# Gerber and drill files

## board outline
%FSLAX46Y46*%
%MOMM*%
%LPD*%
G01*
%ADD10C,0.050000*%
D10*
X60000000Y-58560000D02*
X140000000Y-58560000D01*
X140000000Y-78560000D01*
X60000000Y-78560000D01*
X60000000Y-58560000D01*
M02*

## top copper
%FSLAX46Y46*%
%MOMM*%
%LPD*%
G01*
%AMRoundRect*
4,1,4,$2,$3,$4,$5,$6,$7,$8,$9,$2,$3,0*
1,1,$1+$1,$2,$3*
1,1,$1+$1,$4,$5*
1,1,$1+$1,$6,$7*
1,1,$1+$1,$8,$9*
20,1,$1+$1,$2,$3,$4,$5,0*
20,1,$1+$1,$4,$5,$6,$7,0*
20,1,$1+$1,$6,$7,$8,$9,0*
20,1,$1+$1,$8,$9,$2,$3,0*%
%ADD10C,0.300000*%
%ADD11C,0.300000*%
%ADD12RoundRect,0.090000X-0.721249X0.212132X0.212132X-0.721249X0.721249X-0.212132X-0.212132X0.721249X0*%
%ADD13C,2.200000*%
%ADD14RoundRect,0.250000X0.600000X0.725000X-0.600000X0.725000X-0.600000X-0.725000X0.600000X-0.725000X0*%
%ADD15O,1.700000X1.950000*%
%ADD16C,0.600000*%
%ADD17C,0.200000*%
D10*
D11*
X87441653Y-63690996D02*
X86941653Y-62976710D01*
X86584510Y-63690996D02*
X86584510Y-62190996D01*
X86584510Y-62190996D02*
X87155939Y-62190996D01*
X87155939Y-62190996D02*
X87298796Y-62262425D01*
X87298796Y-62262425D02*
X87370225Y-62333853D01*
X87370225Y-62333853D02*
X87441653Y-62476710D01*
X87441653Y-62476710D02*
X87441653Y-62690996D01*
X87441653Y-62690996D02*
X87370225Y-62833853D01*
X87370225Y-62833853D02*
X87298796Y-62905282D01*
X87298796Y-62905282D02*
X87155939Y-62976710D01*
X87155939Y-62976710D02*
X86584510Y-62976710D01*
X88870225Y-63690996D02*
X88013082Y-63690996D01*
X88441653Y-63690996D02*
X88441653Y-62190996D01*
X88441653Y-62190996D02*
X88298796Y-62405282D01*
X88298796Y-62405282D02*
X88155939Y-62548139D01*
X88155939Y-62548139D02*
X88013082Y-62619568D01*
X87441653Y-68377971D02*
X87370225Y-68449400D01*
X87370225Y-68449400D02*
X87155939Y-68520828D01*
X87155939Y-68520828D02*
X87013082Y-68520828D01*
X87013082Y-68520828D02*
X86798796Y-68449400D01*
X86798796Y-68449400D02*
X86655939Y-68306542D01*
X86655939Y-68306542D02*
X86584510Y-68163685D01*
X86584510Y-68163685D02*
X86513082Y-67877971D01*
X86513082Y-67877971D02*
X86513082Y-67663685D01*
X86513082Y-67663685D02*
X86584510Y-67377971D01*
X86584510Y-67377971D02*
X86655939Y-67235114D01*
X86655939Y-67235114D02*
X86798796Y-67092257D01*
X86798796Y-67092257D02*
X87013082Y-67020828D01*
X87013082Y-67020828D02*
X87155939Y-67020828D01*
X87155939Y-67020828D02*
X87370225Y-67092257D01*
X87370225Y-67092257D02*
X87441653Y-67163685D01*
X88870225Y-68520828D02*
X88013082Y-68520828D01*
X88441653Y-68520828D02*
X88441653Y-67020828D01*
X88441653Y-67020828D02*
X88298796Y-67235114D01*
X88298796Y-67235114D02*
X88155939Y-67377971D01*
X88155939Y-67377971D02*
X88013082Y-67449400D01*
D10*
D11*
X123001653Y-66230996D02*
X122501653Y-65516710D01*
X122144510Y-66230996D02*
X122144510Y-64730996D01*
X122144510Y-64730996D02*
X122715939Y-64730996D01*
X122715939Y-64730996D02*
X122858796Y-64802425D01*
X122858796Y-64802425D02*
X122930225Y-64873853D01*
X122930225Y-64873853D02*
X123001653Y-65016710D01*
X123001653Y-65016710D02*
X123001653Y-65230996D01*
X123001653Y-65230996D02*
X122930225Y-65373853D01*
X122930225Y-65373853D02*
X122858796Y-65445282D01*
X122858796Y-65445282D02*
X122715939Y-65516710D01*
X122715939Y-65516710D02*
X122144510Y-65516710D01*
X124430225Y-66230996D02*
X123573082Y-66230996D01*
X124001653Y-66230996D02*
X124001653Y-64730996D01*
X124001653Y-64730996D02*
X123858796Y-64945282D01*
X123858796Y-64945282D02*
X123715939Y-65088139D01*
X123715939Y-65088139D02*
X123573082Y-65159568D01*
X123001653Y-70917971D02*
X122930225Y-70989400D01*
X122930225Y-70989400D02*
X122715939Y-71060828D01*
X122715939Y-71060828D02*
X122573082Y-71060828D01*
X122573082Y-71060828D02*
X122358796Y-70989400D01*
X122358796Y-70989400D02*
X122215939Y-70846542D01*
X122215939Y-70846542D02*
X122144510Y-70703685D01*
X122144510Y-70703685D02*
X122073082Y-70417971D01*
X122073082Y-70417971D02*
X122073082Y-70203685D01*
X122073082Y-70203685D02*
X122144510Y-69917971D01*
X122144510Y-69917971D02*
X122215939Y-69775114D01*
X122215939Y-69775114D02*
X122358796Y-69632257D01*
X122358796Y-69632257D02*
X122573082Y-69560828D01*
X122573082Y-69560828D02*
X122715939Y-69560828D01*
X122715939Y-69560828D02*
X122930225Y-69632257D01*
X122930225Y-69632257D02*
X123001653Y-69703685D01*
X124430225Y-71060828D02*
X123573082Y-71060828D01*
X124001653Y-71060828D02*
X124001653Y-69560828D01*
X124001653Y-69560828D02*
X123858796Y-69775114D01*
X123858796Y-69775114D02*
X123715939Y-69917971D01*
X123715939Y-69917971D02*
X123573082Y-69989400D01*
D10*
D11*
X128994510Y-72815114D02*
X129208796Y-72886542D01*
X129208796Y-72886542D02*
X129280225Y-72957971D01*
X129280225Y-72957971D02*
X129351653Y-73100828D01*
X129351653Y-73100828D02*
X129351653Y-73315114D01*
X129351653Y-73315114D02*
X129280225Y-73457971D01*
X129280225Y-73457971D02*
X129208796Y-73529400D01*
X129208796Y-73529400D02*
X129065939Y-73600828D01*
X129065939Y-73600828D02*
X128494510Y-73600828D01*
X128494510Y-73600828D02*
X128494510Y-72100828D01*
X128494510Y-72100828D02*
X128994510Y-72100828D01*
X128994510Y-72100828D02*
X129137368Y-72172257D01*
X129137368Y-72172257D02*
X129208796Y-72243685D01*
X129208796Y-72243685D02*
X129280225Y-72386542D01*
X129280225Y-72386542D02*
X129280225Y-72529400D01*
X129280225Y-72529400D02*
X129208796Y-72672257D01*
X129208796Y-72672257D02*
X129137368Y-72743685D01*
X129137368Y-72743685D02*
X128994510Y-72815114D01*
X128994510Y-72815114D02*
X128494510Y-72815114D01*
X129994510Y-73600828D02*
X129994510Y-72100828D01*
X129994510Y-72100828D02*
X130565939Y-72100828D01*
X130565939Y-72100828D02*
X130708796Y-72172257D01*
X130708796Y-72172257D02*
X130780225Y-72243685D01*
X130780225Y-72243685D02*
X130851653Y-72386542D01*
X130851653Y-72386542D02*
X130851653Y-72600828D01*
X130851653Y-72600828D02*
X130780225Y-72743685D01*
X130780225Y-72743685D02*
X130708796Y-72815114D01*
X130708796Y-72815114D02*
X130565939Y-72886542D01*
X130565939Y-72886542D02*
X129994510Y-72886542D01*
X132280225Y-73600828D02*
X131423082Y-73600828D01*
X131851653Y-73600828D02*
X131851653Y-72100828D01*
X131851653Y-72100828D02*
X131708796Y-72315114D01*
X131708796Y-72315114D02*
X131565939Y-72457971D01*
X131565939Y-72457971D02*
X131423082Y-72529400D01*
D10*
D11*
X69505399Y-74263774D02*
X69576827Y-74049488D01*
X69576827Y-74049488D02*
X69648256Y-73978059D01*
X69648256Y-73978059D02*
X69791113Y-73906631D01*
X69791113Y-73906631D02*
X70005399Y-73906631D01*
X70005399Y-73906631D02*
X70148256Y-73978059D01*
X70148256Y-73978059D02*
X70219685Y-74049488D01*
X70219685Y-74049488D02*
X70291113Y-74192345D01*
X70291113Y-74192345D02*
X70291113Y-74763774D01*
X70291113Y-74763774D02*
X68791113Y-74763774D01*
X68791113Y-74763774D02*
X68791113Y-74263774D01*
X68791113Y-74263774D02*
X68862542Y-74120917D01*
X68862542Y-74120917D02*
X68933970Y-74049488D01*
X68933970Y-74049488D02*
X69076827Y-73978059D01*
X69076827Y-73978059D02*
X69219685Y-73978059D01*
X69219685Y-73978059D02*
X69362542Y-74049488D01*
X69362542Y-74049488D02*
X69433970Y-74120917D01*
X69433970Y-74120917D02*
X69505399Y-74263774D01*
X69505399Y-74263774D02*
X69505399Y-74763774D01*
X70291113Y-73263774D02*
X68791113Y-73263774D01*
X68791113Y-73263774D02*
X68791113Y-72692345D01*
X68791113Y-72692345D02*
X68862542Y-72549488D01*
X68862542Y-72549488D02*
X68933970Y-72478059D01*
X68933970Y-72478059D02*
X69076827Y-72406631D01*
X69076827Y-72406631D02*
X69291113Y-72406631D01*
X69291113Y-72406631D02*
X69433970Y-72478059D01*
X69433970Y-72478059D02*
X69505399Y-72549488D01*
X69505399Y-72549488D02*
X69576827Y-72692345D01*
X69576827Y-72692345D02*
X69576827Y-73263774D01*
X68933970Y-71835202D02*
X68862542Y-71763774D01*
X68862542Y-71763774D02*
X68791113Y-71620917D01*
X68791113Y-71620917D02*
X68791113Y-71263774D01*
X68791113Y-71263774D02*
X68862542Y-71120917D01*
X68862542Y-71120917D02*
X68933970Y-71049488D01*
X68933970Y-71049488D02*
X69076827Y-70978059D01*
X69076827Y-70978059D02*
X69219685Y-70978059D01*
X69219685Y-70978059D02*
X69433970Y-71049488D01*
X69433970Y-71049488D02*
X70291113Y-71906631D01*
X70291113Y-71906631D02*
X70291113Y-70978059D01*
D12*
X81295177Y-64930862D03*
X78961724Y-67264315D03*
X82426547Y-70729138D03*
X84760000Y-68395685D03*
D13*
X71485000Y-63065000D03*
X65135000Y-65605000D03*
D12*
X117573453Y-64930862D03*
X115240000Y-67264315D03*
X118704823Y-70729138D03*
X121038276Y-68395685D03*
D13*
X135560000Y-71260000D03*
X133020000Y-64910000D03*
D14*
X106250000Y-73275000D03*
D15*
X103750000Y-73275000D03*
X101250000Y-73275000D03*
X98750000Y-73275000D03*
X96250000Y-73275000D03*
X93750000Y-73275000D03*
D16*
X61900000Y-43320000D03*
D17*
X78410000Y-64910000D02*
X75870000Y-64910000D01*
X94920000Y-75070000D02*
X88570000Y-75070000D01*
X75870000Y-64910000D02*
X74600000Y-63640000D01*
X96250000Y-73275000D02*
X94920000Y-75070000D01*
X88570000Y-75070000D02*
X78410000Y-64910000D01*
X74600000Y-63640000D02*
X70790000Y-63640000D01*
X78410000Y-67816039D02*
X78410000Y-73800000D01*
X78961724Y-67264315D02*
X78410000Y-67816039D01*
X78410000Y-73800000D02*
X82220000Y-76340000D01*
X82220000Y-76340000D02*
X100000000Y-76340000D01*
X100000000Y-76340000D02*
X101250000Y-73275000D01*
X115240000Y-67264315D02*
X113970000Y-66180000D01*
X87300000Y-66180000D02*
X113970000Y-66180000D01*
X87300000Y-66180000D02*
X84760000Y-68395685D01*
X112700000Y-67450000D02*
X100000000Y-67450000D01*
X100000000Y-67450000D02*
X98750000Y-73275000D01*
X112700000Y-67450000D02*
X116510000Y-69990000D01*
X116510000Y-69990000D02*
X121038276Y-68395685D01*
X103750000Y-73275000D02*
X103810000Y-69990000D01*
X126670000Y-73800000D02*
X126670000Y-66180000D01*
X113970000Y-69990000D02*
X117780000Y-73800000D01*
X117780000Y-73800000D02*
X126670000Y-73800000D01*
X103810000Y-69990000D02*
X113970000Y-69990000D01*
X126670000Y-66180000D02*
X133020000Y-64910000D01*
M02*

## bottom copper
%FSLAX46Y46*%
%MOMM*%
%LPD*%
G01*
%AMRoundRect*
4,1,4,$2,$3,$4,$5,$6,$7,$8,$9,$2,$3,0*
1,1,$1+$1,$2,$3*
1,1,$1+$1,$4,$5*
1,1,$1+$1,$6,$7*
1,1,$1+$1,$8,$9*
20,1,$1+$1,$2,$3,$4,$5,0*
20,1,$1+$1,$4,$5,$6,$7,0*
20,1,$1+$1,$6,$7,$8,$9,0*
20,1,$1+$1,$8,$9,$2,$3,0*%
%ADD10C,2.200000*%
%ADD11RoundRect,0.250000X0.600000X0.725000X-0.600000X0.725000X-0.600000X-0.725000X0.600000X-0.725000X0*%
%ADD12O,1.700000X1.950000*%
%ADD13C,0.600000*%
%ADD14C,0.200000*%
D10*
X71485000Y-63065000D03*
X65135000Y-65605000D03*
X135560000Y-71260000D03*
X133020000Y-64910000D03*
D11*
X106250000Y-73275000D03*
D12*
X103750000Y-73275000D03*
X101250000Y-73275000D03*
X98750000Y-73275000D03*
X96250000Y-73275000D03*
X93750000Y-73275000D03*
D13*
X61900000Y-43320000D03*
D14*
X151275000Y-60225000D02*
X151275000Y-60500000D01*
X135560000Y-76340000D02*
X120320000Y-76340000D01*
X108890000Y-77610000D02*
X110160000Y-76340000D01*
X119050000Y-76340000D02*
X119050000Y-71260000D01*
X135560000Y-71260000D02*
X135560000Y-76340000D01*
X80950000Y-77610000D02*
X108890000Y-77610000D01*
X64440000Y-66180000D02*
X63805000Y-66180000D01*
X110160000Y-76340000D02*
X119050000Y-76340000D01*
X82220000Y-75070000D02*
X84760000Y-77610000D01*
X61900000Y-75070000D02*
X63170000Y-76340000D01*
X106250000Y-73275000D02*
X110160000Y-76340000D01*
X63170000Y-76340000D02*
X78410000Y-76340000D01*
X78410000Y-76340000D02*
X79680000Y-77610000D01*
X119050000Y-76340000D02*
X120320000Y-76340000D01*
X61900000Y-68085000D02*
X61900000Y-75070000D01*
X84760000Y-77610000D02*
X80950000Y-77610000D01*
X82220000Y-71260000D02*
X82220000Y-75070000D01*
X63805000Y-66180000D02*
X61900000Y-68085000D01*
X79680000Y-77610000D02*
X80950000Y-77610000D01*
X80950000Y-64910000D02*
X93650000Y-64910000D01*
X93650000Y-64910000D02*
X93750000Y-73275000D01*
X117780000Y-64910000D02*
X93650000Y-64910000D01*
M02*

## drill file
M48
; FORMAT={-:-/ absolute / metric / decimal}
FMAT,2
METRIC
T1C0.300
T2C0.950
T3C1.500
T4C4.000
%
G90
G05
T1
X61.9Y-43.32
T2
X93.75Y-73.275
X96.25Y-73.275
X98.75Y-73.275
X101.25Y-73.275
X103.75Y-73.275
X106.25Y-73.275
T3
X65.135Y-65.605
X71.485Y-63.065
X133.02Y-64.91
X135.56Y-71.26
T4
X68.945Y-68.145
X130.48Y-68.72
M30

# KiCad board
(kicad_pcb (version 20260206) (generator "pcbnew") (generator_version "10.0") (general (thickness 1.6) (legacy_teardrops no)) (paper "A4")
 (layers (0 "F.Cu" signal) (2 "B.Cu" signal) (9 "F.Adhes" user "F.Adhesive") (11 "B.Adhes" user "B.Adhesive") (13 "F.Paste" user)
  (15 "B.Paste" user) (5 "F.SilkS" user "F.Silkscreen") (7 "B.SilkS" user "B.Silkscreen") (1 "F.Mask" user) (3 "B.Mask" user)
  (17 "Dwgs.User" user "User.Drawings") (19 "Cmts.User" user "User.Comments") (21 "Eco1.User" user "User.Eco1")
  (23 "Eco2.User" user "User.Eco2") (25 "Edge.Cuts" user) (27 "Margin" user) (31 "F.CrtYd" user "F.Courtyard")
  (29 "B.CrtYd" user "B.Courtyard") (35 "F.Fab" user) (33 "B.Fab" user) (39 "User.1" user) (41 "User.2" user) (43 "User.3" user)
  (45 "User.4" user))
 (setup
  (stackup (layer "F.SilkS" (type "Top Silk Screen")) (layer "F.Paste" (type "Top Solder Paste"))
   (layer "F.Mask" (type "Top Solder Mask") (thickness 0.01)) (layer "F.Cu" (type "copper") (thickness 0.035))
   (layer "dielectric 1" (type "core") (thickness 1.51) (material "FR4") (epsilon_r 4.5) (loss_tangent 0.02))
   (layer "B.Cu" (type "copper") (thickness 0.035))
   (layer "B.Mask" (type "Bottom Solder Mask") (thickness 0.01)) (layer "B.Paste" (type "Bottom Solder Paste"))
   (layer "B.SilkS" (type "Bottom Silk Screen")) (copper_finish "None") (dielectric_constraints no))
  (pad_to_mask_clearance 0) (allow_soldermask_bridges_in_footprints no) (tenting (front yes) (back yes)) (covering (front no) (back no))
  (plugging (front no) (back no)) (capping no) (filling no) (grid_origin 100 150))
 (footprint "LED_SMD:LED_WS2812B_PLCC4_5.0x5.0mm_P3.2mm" (layer "F.Cu") (at 81.860862 67.83 -45)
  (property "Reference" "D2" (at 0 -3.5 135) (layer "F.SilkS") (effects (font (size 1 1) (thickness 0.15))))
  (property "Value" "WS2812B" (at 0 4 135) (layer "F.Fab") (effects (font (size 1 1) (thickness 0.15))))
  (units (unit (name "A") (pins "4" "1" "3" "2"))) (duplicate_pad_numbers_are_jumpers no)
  (pad "1" smd roundrect (at -2.45 -1.65 315) (size 1.5 0.9) (layers "F.Cu" "F.Mask" "F.Paste") (roundrect_rratio 0.1) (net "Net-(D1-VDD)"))
  (pad "2" smd roundrect (at -2.45 1.65 315) (size 1.5 0.9) (layers "F.Cu" "F.Mask" "F.Paste") (roundrect_rratio 0.1) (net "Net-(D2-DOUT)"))
  (pad "3" smd roundrect (at 2.45 1.65 315) (size 1.5 0.9) (layers "F.Cu" "F.Mask" "F.Paste") (roundrect_rratio 0.1) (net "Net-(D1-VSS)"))
  (pad "4" smd roundrect (at 2.45 -1.65 315) (size 1.5 0.9) (layers "F.Cu" "F.Mask" "F.Paste") (roundrect_rratio 0.1) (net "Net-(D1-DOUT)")))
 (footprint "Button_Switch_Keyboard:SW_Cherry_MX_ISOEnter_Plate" (layer "F.Cu") (at 71.485 63.065)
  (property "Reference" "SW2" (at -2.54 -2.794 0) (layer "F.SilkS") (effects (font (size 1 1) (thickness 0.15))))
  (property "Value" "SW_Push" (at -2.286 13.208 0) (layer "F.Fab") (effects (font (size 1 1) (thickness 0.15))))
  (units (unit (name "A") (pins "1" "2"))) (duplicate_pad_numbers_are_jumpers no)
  (pad "" np_thru_hole circle (at -2.54 5.08) (size 4 4) (drill 4) (layers "*.Cu" "*.Mask"))
  (pad "1" thru_hole circle (at 0 0) (size 2.2 2.2) (drill 1.5) (layers "*.Cu" "*.Mask") (remove_unused_layers no) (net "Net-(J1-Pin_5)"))
  (pad "2" thru_hole circle (at -6.35 2.54) (size 2.2 2.2) (drill 1.5) (layers "*.Cu" "*.Mask") (remove_unused_layers no)
   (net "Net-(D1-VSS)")))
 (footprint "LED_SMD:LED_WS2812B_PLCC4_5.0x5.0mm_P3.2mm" (layer "F.Cu") (at 118.139138 67.83 -45)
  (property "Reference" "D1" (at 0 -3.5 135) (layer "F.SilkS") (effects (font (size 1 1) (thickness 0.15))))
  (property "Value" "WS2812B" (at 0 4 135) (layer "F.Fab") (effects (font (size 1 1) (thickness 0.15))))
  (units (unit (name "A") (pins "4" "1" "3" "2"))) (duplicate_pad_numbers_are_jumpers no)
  (pad "1" smd roundrect (at -2.45 -1.65 315) (size 1.5 0.9) (layers "F.Cu" "F.Mask" "F.Paste") (roundrect_rratio 0.1) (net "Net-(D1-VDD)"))
  (pad "2" smd roundrect (at -2.45 1.65 315) (size 1.5 0.9) (layers "F.Cu" "F.Mask" "F.Paste") (roundrect_rratio 0.1) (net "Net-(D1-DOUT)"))
  (pad "3" smd roundrect (at 2.45 1.65 315) (size 1.5 0.9) (layers "F.Cu" "F.Mask" "F.Paste") (roundrect_rratio 0.1) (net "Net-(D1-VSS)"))
  (pad "4" smd roundrect (at 2.45 -1.65 315) (size 1.5 0.9) (layers "F.Cu" "F.Mask" "F.Paste") (roundrect_rratio 0.1) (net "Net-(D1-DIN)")))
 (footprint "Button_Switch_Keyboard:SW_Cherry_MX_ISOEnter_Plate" (layer "F.Cu") (at 135.56 71.26 -90)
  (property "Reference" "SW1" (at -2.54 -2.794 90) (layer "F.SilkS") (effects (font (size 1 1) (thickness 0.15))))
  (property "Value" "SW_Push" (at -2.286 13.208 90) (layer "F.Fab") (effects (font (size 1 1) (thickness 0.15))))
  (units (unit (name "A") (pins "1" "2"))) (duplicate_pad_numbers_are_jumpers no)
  (pad "" np_thru_hole circle (at -2.54 5.08 270) (size 4 4) (drill 4) (layers "*.Cu" "*.Mask"))
  (pad "1" thru_hole circle (at 0 0 270) (size 2.2 2.2) (drill 1.5) (layers "*.Cu" "*.Mask") (remove_unused_layers no) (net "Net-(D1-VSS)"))
  (pad "2" thru_hole circle (at -6.35 2.54 270) (size 2.2 2.2) (drill 1.5) (layers "*.Cu" "*.Mask") (remove_unused_layers no)
   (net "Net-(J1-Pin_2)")))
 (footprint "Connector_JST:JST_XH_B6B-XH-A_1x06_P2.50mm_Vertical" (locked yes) (layer "B.Cu") (at 106.25 73.275 180)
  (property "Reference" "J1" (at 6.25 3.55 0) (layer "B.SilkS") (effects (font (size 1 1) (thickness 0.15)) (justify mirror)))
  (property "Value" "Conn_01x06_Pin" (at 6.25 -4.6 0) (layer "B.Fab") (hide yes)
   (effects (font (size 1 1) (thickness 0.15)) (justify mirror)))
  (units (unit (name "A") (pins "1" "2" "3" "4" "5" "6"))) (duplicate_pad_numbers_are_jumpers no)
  (pad "1" thru_hole roundrect (at 0 0 180) (size 1.7 1.95) (drill 0.95) (layers "*.Cu" "*.Mask") (remove_unused_layers no)
   (roundrect_rratio 0.147059) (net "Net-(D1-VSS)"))
  (pad "2" thru_hole oval (at 2.5 0 180) (size 1.7 1.95) (drill 0.95) (layers "*.Cu" "*.Mask") (remove_unused_layers no)
   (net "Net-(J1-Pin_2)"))
  (pad "3" thru_hole oval (at 5 0 180) (size 1.7 1.95) (drill 0.95) (layers "*.Cu" "*.Mask") (remove_unused_layers no) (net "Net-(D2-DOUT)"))
  (pad "4" thru_hole oval (at 7.5 0 180) (size 1.7 1.95) (drill 0.95) (layers "*.Cu" "*.Mask") (remove_unused_layers no)
   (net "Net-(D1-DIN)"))
  (pad "5" thru_hole oval (at 10 0 180) (size 1.7 1.95) (drill 0.95) (layers "*.Cu" "*.Mask") (remove_unused_layers no)
   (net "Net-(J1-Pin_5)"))
  (pad "6" thru_hole oval (at 12.5 0 180) (size 1.7 1.95) (drill 0.95) (layers "*.Cu" "*.Mask") (remove_unused_layers no)
   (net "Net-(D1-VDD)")))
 (gr_rect (start 60 58.56) (end 140 78.56) (stroke (width 0.05) (type solid)) (fill no) (layer "Edge.Cuts"))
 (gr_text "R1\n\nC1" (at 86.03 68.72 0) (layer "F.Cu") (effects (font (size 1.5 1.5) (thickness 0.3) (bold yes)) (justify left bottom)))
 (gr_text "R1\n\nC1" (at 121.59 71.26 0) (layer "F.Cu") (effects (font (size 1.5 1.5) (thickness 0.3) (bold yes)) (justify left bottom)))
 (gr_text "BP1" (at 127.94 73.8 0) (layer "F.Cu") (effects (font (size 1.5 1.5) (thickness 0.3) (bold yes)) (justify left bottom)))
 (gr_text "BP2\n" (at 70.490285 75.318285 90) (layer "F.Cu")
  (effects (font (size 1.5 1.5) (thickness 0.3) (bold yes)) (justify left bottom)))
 (via (at 61.9 43.32) (size 0.6) (drill 0.3) (layers "F.Cu" "B.Cu") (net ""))
 (segment (start 151.275 60.225) (end 151.275 60.5) (width 0.2) (layer "B.Cu") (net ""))
 (segment (start 78.41 64.91) (end 75.87 64.91) (width 0.2) (layer "F.Cu") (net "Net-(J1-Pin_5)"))
 (segment (start 94.92 75.07) (end 88.57 75.07) (width 0.2) (layer "F.Cu") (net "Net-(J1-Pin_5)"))
 (segment (start 75.87 64.91) (end 74.6 63.64) (width 0.2) (layer "F.Cu") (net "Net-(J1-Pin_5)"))
 (segment (start 96.25 73.275) (end 94.92 75.07) (width 0.2) (layer "F.Cu") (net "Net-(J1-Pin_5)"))
 (segment (start 88.57 75.07) (end 78.41 64.91) (width 0.2) (layer "F.Cu") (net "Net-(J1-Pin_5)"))
 (segment (start 74.6 63.64) (end 70.79 63.64) (width 0.2) (layer "F.Cu") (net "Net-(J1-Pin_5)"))
 (segment (start 135.56 76.34) (end 120.32 76.34) (width 0.2) (layer "B.Cu") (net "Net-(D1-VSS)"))
 (segment (start 108.89 77.61) (end 110.16 76.34) (width 0.2) (locked yes) (layer "B.Cu") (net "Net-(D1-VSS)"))
 (segment (start 119.05 76.34) (end 119.05 71.26) (width 0.2) (layer "B.Cu") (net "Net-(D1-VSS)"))
 (segment (start 135.56 71.26) (end 135.56 76.34) (width 0.2) (layer "B.Cu") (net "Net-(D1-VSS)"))
 (segment (start 80.95 77.61) (end 108.89 77.61) (width 0.2) (locked yes) (layer "B.Cu") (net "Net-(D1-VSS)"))
 (segment (start 64.44 66.18) (end 63.805 66.18) (width 0.2) (layer "B.Cu") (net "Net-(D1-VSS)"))
 (segment (start 110.16 76.34) (end 119.05 76.34) (width 0.2) (locked yes) (layer "B.Cu") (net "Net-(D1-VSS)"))
 (segment (start 82.22 75.07) (end 84.76 77.61) (width 0.2) (layer "B.Cu") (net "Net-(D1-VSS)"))
 (segment (start 61.9 75.07) (end 63.17 76.34) (width 0.2) (layer "B.Cu") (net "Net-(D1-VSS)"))
 (segment (start 106.25 73.275) (end 110.16 76.34) (width 0.2) (locked yes) (layer "B.Cu") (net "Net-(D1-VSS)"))
 (segment (start 63.17 76.34) (end 78.41 76.34) (width 0.2) (layer "B.Cu") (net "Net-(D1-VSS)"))
 (segment (start 78.41 76.34) (end 79.68 77.61) (width 0.2) (layer "B.Cu") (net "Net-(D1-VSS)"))
 (segment (start 119.05 76.34) (end 120.32 76.34) (width 0.2) (locked yes) (layer "B.Cu") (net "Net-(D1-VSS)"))
 (segment (start 61.9 68.085) (end 61.9 75.07) (width 0.2) (layer "B.Cu") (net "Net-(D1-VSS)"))
 (segment (start 84.76 77.61) (end 80.95 77.61) (width 0.2) (layer "B.Cu") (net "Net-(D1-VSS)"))
 (segment (start 82.22 71.26) (end 82.22 75.07) (width 0.2) (layer "B.Cu") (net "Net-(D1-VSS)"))
 (segment (start 63.805 66.18) (end 61.9 68.085) (width 0.2) (layer "B.Cu") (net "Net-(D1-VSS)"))
 (segment (start 79.68 77.61) (end 80.95 77.61) (width 0.2) (layer "B.Cu") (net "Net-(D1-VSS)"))
 (segment (start 80.95 64.91) (end 93.65 64.91) (width 0.2) (layer "B.Cu") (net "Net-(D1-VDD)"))
 (segment (start 93.65 64.91) (end 93.75 73.275) (width 0.2) (layer "B.Cu") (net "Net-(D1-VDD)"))
 (segment (start 117.78 64.91) (end 93.65 64.91) (width 0.2) (layer "B.Cu") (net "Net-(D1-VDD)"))
 (segment (start 78.41 67.816039) (end 78.41 73.8) (width 0.2) (layer "F.Cu") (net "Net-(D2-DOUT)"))
 (segment (start 78.961724 67.264315) (end 78.41 67.816039) (width 0.2) (layer "F.Cu") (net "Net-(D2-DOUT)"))
 (segment (start 78.41 73.8) (end 82.22 76.34) (width 0.2) (layer "F.Cu") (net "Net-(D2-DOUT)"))
 (segment (start 82.22 76.34) (end 100 76.34) (width 0.2) (layer "F.Cu") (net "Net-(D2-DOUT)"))
 (segment (start 100 76.34) (end 101.25 73.275) (width 0.2) (layer "F.Cu") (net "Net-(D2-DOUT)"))
 (segment (start 115.24 67.264315) (end 113.97 66.18) (width 0.2) (layer "F.Cu") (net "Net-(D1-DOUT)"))
 (segment (start 87.3 66.18) (end 113.97 66.18) (width 0.2) (layer "F.Cu") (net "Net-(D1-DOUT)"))
 (segment (start 87.3 66.18) (end 84.76 68.395685) (width 0.2) (layer "F.Cu") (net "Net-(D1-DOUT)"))
 (segment (start 112.7 67.45) (end 100 67.45) (width 0.2) (layer "F.Cu") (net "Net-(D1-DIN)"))
 (segment (start 100 67.45) (end 98.75 73.275) (width 0.2) (layer "F.Cu") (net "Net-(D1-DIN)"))
 (segment (start 112.7 67.45) (end 116.51 69.99) (width 0.2) (layer "F.Cu") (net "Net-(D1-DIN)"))
 (segment (start 116.51 69.99) (end 121.038276 68.395685) (width 0.2) (layer "F.Cu") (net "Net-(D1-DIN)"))
 (segment (start 103.75 73.275) (end 103.81 69.99) (width 0.2) (layer "F.Cu") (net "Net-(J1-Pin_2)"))
 (segment (start 126.67 73.8) (end 126.67 66.18) (width 0.2) (layer "F.Cu") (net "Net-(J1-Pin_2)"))
 (segment (start 113.97 69.99) (end 117.78 73.8) (width 0.2) (layer "F.Cu") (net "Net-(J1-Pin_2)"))
 (segment (start 117.78 73.8) (end 126.67 73.8) (width 0.2) (layer "F.Cu") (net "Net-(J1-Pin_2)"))
 (segment (start 103.81 69.99) (end 113.97 69.99) (width 0.2) (layer "F.Cu") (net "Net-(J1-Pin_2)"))
 (segment (start 126.67 66.18) (end 133.02 64.91) (width 0.2) (layer "F.Cu") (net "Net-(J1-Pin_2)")))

